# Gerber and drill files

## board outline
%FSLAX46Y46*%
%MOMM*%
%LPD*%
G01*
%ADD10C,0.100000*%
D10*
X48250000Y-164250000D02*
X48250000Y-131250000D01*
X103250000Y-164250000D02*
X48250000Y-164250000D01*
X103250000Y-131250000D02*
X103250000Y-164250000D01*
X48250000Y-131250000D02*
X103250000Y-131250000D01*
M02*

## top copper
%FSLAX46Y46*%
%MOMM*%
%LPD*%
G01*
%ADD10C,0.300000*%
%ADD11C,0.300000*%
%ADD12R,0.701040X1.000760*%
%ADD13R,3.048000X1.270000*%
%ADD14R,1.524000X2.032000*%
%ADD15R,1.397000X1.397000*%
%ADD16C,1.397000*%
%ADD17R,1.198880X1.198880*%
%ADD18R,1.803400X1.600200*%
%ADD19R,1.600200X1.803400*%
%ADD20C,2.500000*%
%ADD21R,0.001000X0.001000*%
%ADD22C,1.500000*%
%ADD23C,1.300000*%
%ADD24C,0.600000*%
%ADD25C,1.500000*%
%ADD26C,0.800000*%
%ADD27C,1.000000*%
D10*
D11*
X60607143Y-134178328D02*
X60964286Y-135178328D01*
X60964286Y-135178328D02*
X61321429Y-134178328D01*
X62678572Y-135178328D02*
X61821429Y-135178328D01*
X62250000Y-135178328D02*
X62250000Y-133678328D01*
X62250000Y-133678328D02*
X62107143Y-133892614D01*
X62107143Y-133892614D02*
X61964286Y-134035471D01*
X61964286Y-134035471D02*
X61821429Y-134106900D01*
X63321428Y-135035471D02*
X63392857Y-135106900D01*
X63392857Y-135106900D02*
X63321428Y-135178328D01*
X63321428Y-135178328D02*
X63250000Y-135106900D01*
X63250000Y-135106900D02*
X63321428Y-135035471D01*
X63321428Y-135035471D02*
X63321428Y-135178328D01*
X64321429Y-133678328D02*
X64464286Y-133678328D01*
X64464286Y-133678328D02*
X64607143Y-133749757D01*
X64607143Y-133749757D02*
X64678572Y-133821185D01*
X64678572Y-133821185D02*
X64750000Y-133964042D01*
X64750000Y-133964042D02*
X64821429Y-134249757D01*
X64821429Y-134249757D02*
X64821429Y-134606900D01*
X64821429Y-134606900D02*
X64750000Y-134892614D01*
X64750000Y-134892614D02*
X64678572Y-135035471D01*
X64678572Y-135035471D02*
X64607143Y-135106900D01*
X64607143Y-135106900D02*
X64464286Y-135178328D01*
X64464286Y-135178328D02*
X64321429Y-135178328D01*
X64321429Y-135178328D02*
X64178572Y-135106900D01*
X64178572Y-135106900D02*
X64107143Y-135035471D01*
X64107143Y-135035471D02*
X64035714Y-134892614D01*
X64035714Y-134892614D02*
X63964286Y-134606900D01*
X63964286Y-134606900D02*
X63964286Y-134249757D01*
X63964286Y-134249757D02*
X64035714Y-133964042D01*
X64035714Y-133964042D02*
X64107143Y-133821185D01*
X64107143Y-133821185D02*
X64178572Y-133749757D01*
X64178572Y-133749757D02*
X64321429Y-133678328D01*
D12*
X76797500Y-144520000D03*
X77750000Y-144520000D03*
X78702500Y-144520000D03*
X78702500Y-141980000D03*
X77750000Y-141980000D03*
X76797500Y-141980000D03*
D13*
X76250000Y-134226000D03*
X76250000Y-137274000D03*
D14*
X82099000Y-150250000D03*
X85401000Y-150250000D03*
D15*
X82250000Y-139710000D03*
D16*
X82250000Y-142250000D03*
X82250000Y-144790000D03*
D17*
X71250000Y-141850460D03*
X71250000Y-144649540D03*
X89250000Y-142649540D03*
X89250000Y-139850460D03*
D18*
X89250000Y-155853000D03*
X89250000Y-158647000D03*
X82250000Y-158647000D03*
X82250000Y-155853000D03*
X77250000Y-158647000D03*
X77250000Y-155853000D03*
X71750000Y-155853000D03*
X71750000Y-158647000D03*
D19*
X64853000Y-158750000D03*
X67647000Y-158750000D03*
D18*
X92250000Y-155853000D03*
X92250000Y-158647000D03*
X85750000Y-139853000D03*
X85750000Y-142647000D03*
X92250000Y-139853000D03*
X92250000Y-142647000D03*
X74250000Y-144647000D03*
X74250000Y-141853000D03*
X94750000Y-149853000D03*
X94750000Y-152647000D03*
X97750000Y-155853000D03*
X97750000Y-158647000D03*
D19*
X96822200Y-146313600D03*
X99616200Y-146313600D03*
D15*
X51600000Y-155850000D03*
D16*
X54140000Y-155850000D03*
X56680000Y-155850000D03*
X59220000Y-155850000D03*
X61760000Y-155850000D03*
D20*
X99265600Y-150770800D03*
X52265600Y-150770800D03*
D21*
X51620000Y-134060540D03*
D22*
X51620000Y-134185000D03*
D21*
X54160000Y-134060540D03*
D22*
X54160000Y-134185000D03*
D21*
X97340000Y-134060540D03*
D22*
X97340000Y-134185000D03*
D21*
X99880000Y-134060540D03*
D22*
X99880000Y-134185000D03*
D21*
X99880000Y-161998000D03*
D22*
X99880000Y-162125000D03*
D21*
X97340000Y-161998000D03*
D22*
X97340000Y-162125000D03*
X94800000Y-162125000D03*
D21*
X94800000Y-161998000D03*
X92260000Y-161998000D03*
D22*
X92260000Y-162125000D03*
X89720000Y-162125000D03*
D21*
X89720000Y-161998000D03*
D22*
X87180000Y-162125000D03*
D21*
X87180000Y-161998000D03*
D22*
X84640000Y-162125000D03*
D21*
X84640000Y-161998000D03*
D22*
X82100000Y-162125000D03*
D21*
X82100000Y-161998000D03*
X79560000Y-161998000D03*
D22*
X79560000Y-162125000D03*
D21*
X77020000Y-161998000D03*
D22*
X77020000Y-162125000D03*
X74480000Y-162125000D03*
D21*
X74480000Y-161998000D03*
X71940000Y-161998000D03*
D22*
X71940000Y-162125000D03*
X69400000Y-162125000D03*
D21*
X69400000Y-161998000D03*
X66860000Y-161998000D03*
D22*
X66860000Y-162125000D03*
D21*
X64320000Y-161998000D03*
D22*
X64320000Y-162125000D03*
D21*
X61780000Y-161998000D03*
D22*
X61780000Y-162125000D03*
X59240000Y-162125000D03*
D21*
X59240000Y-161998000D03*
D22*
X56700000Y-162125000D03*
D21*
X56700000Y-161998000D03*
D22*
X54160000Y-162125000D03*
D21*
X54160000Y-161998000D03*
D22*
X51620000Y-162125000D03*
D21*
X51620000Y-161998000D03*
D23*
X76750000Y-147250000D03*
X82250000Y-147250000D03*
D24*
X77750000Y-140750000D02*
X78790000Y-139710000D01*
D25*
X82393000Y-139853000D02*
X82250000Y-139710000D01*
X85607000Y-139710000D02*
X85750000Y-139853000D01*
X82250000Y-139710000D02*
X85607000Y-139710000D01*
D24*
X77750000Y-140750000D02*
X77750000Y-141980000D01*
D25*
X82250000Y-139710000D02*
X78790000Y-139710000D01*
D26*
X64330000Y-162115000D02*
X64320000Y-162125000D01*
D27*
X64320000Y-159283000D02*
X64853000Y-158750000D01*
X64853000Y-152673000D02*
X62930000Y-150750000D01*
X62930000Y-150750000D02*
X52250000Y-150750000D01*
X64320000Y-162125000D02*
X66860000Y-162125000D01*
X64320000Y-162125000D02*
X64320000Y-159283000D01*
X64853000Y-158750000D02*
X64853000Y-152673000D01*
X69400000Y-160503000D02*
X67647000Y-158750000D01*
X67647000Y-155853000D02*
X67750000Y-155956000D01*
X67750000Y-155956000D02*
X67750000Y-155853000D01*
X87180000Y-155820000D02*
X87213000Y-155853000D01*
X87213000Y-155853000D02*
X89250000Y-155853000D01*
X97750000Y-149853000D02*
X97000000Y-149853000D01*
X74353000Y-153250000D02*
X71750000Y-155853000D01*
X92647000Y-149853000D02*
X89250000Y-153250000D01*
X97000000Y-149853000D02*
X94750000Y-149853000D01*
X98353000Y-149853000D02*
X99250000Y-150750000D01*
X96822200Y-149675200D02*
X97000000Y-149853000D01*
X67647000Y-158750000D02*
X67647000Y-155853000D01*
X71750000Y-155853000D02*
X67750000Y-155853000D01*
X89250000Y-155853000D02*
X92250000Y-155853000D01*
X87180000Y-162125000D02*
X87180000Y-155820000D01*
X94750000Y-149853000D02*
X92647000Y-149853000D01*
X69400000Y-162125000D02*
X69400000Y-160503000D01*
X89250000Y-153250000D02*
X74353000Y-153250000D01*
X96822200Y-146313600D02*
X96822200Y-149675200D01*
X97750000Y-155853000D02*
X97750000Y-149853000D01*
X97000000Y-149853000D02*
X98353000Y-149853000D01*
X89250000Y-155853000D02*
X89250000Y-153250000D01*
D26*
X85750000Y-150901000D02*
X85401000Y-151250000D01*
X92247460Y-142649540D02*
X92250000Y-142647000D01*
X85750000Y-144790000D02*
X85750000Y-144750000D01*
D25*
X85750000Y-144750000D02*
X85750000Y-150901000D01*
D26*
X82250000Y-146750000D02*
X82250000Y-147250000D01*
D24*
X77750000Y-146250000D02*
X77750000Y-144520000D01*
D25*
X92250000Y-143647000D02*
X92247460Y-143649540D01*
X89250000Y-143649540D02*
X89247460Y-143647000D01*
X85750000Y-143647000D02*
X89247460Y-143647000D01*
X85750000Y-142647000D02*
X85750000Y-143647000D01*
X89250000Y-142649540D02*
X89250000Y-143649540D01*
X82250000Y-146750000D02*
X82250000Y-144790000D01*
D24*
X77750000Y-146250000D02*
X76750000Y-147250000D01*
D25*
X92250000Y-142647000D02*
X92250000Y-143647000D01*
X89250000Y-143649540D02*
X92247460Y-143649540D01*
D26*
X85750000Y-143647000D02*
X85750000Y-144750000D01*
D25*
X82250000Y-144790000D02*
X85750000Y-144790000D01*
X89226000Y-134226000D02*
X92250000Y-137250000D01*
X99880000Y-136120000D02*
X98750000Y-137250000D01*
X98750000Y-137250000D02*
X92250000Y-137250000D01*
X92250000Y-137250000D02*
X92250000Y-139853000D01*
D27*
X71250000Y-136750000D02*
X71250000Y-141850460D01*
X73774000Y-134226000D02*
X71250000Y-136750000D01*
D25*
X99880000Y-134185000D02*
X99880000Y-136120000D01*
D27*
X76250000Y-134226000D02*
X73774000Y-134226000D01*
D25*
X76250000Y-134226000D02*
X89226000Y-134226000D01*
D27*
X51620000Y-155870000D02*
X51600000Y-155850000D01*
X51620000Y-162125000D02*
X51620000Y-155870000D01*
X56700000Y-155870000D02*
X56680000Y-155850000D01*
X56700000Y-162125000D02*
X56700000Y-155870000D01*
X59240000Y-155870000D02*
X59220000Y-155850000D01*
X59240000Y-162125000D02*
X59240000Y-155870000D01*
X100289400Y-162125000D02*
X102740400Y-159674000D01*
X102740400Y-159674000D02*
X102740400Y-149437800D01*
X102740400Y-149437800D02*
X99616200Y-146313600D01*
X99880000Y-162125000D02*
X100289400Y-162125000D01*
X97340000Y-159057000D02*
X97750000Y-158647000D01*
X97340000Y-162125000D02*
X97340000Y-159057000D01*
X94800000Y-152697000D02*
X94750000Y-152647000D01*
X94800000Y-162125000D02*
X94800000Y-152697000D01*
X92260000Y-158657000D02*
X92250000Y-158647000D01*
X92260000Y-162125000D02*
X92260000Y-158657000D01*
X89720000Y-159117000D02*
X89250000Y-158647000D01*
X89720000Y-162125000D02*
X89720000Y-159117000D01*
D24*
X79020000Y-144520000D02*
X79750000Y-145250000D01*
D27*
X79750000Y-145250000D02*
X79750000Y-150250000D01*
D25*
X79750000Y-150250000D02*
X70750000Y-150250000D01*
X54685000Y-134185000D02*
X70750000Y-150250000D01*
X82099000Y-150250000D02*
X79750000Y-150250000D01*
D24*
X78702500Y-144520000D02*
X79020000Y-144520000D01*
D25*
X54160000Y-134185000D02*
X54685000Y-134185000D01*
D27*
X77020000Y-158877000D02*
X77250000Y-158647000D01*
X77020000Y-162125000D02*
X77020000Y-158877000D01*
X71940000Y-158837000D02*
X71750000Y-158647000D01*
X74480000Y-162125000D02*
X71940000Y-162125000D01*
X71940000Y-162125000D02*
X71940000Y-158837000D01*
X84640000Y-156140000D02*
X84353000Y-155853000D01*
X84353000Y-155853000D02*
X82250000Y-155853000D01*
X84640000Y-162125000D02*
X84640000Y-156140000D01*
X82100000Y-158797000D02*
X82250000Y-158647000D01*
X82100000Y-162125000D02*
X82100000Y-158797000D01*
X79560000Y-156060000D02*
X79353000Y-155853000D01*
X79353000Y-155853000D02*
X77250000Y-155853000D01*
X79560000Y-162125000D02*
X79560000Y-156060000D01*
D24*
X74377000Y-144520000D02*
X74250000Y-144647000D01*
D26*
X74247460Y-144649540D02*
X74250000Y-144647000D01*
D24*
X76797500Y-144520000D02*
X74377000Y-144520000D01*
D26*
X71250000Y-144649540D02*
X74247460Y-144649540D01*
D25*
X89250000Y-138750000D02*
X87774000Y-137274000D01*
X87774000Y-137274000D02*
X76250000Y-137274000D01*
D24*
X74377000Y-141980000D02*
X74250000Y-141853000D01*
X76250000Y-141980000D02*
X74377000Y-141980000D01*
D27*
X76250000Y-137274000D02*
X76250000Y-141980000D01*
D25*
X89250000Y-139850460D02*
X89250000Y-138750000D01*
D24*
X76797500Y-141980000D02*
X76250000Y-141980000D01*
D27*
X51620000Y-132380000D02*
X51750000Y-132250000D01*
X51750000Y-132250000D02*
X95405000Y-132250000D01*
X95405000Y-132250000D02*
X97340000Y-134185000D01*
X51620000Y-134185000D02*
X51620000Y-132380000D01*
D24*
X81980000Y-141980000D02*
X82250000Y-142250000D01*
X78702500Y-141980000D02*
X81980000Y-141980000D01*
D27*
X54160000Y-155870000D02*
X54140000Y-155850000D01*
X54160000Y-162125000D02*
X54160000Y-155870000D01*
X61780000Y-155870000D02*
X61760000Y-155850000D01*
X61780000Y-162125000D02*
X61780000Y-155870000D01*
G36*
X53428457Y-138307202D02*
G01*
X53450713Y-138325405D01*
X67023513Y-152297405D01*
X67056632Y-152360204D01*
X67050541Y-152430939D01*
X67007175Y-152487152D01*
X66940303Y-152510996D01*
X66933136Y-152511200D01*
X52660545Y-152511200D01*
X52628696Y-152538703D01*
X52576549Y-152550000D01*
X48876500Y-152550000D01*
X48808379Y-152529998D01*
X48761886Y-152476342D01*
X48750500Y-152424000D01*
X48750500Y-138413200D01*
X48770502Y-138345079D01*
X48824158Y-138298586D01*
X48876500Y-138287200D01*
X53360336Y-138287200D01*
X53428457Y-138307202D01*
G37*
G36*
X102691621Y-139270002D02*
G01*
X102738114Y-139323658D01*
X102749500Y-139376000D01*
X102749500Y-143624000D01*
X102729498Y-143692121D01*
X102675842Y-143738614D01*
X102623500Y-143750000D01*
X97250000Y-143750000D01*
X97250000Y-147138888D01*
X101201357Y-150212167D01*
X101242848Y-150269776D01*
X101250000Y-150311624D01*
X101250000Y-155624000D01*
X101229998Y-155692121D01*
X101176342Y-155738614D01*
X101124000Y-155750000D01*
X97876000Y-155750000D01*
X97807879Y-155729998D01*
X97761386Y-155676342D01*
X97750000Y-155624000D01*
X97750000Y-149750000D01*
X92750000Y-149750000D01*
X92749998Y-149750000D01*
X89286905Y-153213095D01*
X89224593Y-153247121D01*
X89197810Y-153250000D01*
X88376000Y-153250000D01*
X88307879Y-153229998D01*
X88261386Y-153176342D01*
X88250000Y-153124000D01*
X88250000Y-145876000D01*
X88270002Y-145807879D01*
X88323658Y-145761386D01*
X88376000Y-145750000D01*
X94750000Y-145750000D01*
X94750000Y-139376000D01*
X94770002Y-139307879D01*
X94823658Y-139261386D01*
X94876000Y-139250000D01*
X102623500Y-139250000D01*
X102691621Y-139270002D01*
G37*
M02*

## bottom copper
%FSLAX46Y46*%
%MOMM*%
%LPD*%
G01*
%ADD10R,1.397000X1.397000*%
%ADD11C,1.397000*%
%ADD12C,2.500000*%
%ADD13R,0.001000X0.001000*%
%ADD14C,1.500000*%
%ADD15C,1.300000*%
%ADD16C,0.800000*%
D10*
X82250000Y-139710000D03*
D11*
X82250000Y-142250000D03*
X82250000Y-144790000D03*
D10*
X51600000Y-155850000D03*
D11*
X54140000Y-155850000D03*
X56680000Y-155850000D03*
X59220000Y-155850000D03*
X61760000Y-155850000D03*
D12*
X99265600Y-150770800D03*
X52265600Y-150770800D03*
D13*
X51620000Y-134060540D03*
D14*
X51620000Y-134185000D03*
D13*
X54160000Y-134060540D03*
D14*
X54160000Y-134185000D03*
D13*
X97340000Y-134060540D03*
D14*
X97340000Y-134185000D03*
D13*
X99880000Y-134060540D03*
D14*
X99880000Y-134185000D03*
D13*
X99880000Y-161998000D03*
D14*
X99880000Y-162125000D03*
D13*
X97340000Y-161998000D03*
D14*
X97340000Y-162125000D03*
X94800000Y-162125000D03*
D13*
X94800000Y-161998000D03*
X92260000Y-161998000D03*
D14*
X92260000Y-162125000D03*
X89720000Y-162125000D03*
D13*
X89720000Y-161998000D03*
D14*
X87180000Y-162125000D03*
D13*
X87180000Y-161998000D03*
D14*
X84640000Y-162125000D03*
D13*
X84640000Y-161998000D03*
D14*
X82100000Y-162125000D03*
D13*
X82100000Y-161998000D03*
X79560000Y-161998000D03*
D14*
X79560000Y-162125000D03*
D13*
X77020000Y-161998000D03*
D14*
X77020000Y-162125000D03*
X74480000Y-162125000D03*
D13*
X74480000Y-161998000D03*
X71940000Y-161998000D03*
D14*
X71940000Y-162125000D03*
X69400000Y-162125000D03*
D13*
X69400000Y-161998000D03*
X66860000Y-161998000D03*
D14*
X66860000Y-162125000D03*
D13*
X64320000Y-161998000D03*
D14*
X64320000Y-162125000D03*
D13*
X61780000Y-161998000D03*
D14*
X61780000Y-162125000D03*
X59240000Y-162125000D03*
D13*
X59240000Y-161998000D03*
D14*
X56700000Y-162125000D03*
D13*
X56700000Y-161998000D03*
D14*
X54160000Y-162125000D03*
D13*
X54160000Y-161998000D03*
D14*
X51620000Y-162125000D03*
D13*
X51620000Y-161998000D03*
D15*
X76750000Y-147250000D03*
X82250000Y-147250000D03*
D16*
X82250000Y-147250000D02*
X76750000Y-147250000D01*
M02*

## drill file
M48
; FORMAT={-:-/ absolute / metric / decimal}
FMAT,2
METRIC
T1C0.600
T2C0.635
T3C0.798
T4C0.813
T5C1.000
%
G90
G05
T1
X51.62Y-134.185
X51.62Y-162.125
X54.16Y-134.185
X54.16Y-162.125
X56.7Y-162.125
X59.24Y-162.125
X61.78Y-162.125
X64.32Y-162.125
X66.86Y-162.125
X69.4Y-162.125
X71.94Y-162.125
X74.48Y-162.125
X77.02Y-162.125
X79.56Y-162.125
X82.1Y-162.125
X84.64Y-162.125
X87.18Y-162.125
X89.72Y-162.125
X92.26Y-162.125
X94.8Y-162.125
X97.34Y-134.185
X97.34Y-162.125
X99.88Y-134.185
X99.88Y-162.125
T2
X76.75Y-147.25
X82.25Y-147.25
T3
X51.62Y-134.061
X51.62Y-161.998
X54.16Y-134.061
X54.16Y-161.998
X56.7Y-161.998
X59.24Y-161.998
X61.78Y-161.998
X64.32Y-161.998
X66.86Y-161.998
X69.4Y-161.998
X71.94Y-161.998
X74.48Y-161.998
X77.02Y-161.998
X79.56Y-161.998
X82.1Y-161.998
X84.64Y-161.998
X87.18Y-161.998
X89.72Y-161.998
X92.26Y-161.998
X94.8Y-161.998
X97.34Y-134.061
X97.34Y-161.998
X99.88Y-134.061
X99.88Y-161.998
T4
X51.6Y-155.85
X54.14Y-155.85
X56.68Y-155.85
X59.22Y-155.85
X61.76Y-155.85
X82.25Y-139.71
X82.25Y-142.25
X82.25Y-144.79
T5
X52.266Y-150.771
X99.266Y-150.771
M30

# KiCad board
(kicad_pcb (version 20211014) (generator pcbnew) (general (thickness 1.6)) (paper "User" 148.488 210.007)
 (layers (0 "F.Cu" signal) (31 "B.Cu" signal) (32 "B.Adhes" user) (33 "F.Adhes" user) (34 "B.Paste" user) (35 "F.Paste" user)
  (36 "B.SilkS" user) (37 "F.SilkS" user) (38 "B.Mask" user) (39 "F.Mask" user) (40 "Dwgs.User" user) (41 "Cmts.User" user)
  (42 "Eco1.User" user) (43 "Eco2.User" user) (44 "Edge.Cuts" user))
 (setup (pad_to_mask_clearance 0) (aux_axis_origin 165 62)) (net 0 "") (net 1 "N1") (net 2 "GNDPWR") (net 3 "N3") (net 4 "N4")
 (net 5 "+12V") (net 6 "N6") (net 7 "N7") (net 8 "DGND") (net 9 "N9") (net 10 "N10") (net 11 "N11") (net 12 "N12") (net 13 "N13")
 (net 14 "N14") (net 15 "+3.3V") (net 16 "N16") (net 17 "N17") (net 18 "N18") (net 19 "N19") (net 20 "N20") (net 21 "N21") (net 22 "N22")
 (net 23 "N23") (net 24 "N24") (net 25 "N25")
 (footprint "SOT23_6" (layer "F.Cu") (at 77.75 143.25)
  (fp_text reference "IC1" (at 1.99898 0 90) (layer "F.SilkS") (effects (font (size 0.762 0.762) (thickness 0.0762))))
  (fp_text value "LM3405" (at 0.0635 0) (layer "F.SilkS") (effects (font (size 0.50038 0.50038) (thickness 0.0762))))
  (pad "1" smd rect locked (at -0.9525 1.27) (size 0.70104 1.00076) (layers "F.Cu" "F.Paste" "F.Mask") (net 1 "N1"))
  (pad "2" smd rect locked (at 0 1.27) (size 0.70104 1.00076) (layers "F.Cu" "F.Paste" "F.Mask") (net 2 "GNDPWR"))
  (pad "3" smd rect locked (at 0.9525 1.27) (size 0.70104 1.00076) (layers "F.Cu" "F.Paste" "F.Mask") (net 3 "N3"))
  (pad "4" smd rect locked (at 0.9525 -1.27) (size 0.70104 1.00076) (layers "F.Cu" "F.Paste" "F.Mask") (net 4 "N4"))
  (pad "5" smd rect locked (at 0 -1.27) (size 0.70104 1.00076) (layers "F.Cu" "F.Paste" "F.Mask") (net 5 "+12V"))
  (pad "6" smd rect locked (at -0.9525 -1.27) (size 0.70104 1.00076) (layers "F.Cu" "F.Paste" "F.Mask") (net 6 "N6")))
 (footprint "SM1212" (layer "F.Cu") (at 76.25 135.75 -90)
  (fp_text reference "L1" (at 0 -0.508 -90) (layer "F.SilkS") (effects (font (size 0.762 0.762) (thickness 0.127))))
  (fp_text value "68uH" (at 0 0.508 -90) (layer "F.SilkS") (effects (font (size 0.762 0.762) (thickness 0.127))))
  (pad "1" smd rect locked (at -1.524 0 270) (size 1.27 3.048) (layers "F.Cu" "F.Paste" "F.Mask") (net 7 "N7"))
  (pad "2" smd rect locked (at 1.524 0 270) (size 1.27 3.048) (layers "F.Cu" "F.Paste" "F.Mask") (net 6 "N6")))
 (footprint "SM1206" (layer "F.Cu") (at 83.75 150.25)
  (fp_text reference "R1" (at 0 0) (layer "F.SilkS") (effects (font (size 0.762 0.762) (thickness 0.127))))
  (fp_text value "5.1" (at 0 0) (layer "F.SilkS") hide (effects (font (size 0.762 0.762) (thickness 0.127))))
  (pad "1" smd rect locked (at -1.651 0) (size 1.524 2.032) (layers "F.Cu" "F.Paste" "F.Mask") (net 3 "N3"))
  (pad "2" smd rect locked (at 1.651 0) (size 1.524 2.032) (layers "F.Cu" "F.Paste" "F.Mask") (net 2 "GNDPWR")))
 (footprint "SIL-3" (layer "F.Cu") (at 82.25 142.25 -90)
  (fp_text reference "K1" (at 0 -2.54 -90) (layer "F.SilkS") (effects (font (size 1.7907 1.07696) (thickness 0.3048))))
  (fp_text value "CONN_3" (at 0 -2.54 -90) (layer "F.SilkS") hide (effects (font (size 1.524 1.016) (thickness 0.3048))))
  (pad "1" thru_hole rect locked (at -2.54 0 270) (size 1.397 1.397) (drill 0.8128) (layers *.Cu *.Mask "F.SilkS") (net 5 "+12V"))
  (pad "2" thru_hole circle locked (at 0 0 270) (size 1.397 1.397) (drill 0.8128) (layers *.Cu *.Mask "F.SilkS") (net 4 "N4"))
  (pad "3" thru_hole circle locked (at 2.54 0 270) (size 1.397 1.397) (drill 0.8128) (layers *.Cu *.Mask "F.SilkS") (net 2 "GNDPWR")))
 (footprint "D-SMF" (layer "F.Cu") (at 71.25 143.25 -90)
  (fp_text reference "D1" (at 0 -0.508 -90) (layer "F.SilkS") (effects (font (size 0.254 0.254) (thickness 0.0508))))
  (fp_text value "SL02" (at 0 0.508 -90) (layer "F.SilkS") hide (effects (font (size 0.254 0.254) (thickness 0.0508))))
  (pad "1" smd rect locked (at -1.39954 0 270) (size 1.19888 1.19888) (layers "F.Cu" "F.Paste" "F.Mask") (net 7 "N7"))
  (pad "2" smd rect locked (at 1.39954 0 270) (size 1.19888 1.19888) (layers "F.Cu" "F.Paste" "F.Mask") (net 1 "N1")))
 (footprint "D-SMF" (layer "F.Cu") (at 89.25 141.25 90)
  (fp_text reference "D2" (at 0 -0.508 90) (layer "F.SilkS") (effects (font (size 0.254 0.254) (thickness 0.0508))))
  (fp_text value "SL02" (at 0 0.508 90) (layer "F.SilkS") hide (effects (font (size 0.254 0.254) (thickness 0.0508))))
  (pad "1" smd rect locked (at -1.39954 0 90) (size 1.19888 1.19888) (layers "F.Cu" "F.Paste" "F.Mask") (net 2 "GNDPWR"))
  (pad "2" smd rect locked (at 1.39954 0 90) (size 1.19888 1.19888) (layers "F.Cu" "F.Paste" "F.Mask") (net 6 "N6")))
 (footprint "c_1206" (layer "F.Cu") (at 89.25 157.25 90)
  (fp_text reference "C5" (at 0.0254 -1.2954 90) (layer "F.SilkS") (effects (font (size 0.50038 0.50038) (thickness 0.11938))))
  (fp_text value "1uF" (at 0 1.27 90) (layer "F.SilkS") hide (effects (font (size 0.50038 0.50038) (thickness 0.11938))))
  (pad "1" smd rect locked (at 1.397 0 90) (size 1.6002 1.8034) (layers "F.Cu" "F.Paste" "F.Mask") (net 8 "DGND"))
  (pad "2" smd rect locked (at -1.397 0 90) (size 1.6002 1.8034) (layers "F.Cu" "F.Paste" "F.Mask") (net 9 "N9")))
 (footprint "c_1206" (layer "F.Cu") (at 82.25 157.25 -90)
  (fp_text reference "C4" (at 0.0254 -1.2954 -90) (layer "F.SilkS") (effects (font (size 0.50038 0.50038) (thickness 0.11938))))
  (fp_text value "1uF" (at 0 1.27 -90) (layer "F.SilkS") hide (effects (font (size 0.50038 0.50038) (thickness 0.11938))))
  (pad "1" smd rect locked (at 1.397 0 270) (size 1.6002 1.8034) (layers "F.Cu" "F.Paste" "F.Mask") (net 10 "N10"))
  (pad "2" smd rect locked (at -1.397 0 270) (size 1.6002 1.8034) (layers "F.Cu" "F.Paste" "F.Mask") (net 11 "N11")))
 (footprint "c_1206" (layer "F.Cu") (at 77.25 157.25 -90)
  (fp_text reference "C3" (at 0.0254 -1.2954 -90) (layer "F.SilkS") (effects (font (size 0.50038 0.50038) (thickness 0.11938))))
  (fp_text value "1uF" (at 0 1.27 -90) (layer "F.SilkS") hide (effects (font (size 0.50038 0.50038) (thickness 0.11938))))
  (pad "1" smd rect locked (at 1.397 0 270) (size 1.6002 1.8034) (layers "F.Cu" "F.Paste" "F.Mask") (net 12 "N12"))
  (pad "2" smd rect locked (at -1.397 0 270) (size 1.6002 1.8034) (layers "F.Cu" "F.Paste" "F.Mask") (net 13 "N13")))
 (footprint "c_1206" (layer "F.Cu") (at 71.75 157.25 90)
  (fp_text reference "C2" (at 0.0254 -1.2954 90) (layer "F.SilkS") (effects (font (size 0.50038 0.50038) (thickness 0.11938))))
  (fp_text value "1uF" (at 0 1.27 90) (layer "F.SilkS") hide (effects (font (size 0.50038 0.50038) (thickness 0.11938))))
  (pad "1" smd rect locked (at 1.397 0 90) (size 1.6002 1.8034) (layers "F.Cu" "F.Paste" "F.Mask") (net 8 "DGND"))
  (pad "2" smd rect locked (at -1.397 0 90) (size 1.6002 1.8034) (layers "F.Cu" "F.Paste" "F.Mask") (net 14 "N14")))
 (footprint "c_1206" (layer "F.Cu") (at 66.25 158.75 180)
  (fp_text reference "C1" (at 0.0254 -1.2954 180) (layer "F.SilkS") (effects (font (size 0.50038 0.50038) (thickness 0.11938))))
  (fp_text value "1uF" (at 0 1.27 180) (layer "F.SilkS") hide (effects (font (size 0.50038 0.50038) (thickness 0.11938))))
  (pad "1" smd rect locked (at 1.397 0 180) (size 1.6002 1.8034) (layers "F.Cu" "F.Paste" "F.Mask") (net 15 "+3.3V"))
  (pad "2" smd rect locked (at -1.397 0 180) (size 1.6002 1.8034) (layers "F.Cu" "F.Paste" "F.Mask") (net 8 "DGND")))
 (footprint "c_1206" (layer "F.Cu") (at 92.25 157.25 90)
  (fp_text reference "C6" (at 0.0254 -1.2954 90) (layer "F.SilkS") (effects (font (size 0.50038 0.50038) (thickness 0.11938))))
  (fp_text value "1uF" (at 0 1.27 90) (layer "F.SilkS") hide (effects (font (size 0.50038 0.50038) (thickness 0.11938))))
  (pad "1" smd rect locked (at 1.397 0 90) (size 1.6002 1.8034) (layers "F.Cu" "F.Paste" "F.Mask") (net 8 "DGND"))
  (pad "2" smd rect locked (at -1.397 0 90) (size 1.6002 1.8034) (layers "F.Cu" "F.Paste" "F.Mask") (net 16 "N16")))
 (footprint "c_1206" (layer "F.Cu") (at 85.75 141.25 90)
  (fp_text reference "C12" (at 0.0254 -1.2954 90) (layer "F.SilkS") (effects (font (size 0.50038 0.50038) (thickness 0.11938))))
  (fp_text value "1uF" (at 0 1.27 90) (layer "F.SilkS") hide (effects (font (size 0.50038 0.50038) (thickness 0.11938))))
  (pad "1" smd rect locked (at 1.397 0 90) (size 1.6002 1.8034) (layers "F.Cu" "F.Paste" "F.Mask") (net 5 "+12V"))
  (pad "2" smd rect locked (at -1.397 0 90) (size 1.6002 1.8034) (layers "F.Cu" "F.Paste" "F.Mask") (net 2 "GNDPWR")))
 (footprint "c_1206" (layer "F.Cu") (at 92.25 141.25 90)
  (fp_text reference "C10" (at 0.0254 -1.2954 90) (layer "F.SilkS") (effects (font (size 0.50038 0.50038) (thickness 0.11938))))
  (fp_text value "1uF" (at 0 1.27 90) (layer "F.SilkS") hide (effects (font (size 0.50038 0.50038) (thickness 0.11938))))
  (pad "1" smd rect locked (at 1.397 0 90) (size 1.6002 1.8034) (layers "F.Cu" "F.Paste" "F.Mask") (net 7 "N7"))
  (pad "2" smd rect locked (at -1.397 0 90) (size 1.6002 1.8034) (layers "F.Cu" "F.Paste" "F.Mask") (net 2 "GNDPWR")))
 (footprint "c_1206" (layer "F.Cu") (at 74.25 143.25 -90)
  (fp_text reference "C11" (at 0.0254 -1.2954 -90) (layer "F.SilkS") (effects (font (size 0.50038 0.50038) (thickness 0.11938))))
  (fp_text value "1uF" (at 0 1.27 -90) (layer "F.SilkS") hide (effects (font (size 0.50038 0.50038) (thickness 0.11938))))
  (pad "1" smd rect locked (at 1.397 0 270) (size 1.6002 1.8034) (layers "F.Cu" "F.Paste" "F.Mask") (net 1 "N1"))
  (pad "2" smd rect locked (at -1.397 0 270) (size 1.6002 1.8034) (layers "F.Cu" "F.Paste" "F.Mask") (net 6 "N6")))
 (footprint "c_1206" (layer "F.Cu") (at 94.75 151.25 90)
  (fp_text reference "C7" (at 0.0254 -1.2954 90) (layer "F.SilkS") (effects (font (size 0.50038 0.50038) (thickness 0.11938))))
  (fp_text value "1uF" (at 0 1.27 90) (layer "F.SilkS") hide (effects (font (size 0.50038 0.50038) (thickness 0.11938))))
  (pad "1" smd rect locked (at 1.397 0 90) (size 1.6002 1.8034) (layers "F.Cu" "F.Paste" "F.Mask") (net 8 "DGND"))
  (pad "2" smd rect locked (at -1.397 0 90) (size 1.6002 1.8034) (layers "F.Cu" "F.Paste" "F.Mask") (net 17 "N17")))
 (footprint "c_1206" (layer "F.Cu") (at 97.75 157.25 90)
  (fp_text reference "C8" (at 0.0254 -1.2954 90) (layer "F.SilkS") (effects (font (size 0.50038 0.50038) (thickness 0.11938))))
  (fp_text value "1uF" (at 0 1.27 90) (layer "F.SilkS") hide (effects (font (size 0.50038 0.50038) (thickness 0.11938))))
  (pad "1" smd rect locked (at 1.397 0 90) (size 1.6002 1.8034) (layers "F.Cu" "F.Paste" "F.Mask") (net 8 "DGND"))
  (pad "2" smd rect locked (at -1.397 0 90) (size 1.6002 1.8034) (layers "F.Cu" "F.Paste" "F.Mask") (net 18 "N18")))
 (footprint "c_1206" (layer "F.Cu") (at 98.2192 146.3136 180)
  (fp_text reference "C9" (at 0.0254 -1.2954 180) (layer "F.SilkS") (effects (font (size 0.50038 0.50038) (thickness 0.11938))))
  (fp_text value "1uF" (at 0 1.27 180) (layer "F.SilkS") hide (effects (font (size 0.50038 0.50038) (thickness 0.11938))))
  (pad "1" smd rect locked (at 1.397 0 180) (size 1.6002 1.8034) (layers "F.Cu" "F.Paste" "F.Mask") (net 8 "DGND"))
  (pad "2" smd rect locked (at -1.397 0 180) (size 1.6002 1.8034) (layers "F.Cu" "F.Paste" "F.Mask") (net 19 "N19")))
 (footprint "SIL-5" (layer "F.Cu") (at 57.95 155.85)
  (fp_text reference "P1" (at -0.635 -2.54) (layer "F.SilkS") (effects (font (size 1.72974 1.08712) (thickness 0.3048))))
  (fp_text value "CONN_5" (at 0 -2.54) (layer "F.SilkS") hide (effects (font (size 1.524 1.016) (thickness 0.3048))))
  (pad "1" thru_hole rect locked (at -6.35 0) (size 1.397 1.397) (drill 0.8128) (layers *.Cu *.Mask "F.SilkS") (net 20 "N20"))
  (pad "2" thru_hole circle locked (at -3.81 0) (size 1.397 1.397) (drill 0.8128) (layers *.Cu *.Mask "F.SilkS") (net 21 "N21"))
  (pad "3" thru_hole circle locked (at -1.27 0) (size 1.397 1.397) (drill 0.8128) (layers *.Cu *.Mask "F.SilkS") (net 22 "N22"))
  (pad "4" thru_hole circle locked (at 1.27 0) (size 1.397 1.397) (drill 0.8128) (layers *.Cu *.Mask "F.SilkS") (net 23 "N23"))
  (pad "5" thru_hole circle locked (at 3.81 0) (size 1.397 1.397) (drill 0.8128) (layers *.Cu *.Mask "F.SilkS") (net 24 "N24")))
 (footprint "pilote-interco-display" (layer "F.Cu") (at 75.7656 146.7708 180)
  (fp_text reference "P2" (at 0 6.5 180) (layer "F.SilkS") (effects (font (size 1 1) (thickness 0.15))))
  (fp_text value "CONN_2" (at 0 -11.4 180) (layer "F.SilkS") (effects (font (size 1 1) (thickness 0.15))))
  (pad "1" thru_hole circle locked (at -23.5 -4 180) (size 2.5 2.5) (drill 1) (layers *.Cu *.Mask "F.SilkS") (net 8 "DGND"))
  (pad "2" thru_hole circle locked (at 23.5 -4 180) (size 2.5 2.5) (drill 1) (layers *.Cu *.Mask "F.SilkS") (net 15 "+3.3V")))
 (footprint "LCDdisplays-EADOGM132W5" (layer "B.Cu") (at 75.75 146.25)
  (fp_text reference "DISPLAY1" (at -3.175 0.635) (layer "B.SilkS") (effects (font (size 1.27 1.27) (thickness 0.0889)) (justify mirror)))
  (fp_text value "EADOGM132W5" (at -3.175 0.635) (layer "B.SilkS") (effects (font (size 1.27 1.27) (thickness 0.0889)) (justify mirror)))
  (pad "1" thru_hole rect locked (at -24.13 -12.18946) (size 1.30556 0) (drill 0.79756) (layers *.Cu "B.Paste" "B.SilkS" "B.Mask")
   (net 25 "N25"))
  (pad "1" thru_hole circle locked (at -24.13 -12.065) (size 1.5 1.5) (drill 0.6) (layers *.Cu *.Mask "B.SilkS") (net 25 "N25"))
  (pad "2" thru_hole rect locked (at -21.59 -12.18946) (size 1.30556 0) (drill 0.79756) (layers *.Cu "B.Paste" "B.SilkS" "B.Mask")
   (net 3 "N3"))
  (pad "2" thru_hole circle locked (at -21.59 -12.065) (size 1.5 1.5) (drill 0.6) (layers *.Cu *.Mask "B.SilkS") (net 3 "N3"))
  (pad "19" thru_hole rect locked (at 21.59 -12.18946) (size 1.30556 0) (drill 0.79756) (layers *.Cu "B.Paste" "B.SilkS" "B.Mask")
   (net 25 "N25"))
  (pad "19" thru_hole circle locked (at 21.59 -12.065) (size 1.5 1.5) (drill 0.6) (layers *.Cu *.Mask "B.SilkS") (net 25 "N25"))
  (pad "20" thru_hole rect locked (at 24.13 -12.18946) (size 1.30556 0) (drill 0.79756) (layers *.Cu "B.Paste" "B.SilkS" "B.Mask")
   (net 7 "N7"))
  (pad "20" thru_hole circle locked (at 24.13 -12.065) (size 1.5 1.5) (drill 0.6) (layers *.Cu *.Mask "B.SilkS") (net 7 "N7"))
  (pad "21" thru_hole rect locked (at 24.13 15.748) (size 1.30556 0) (drill 0.79756) (layers *.Cu "B.Paste" "B.SilkS" "B.Mask")
   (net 19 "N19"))
  (pad "21" thru_hole circle locked (at 24.13 15.875) (size 1.5 1.5) (drill 0.6) (layers *.Cu *.Mask "B.SilkS") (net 19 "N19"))
  (pad "22" thru_hole rect locked (at 21.59 15.748) (size 1.30556 0) (drill 0.79756) (layers *.Cu "B.Paste" "B.SilkS" "B.Mask")
   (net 18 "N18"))
  (pad "22" thru_hole circle locked (at 21.59 15.875) (size 1.5 1.5) (drill 0.6) (layers *.Cu *.Mask "B.SilkS") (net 18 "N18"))
  (pad "23" thru_hole circle locked (at 19.05 15.875) (size 1.5 1.5) (drill 0.6) (layers *.Cu *.Mask "B.SilkS") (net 17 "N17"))
  (pad "23" thru_hole rect locked (at 19.05 15.748) (size 1.30556 0) (drill 0.79756) (layers *.Cu "B.Paste" "B.SilkS" "B.Mask")
   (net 17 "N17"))
  (pad "24" thru_hole rect locked (at 16.51 15.748) (size 1.30556 0) (drill 0.79756) (layers *.Cu "B.Paste" "B.SilkS" "B.Mask")
   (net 16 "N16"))
  (pad "24" thru_hole circle locked (at 16.51 15.875) (size 1.5 1.5) (drill 0.6) (layers *.Cu *.Mask "B.SilkS") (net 16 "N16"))
  (pad "25" thru_hole circle locked (at 13.97 15.875) (size 1.5 1.5) (drill 0.6) (layers *.Cu *.Mask "B.SilkS") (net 9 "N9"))
  (pad "25" thru_hole rect locked (at 13.97 15.748) (size 1.30556 0) (drill 0.79756) (layers *.Cu "B.Paste" "B.SilkS" "B.Mask") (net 9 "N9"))
  (pad "26" thru_hole circle locked (at 11.43 15.875) (size 1.5 1.5) (drill 0.6) (layers *.Cu *.Mask "B.SilkS") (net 8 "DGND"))
  (pad "26" thru_hole rect locked (at 11.43 15.748) (size 1.30556 0) (drill 0.79756) (layers *.Cu "B.Paste" "B.SilkS" "B.Mask")
   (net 8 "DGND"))
  (pad "27" thru_hole circle locked (at 8.89 15.875) (size 1.5 1.5) (drill 0.6) (layers *.Cu *.Mask "B.SilkS") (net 11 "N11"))
  (pad "27" thru_hole rect locked (at 8.89 15.748) (size 1.30556 0) (drill 0.79756) (layers *.Cu "B.Paste" "B.SilkS" "B.Mask")
   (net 11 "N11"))
  (pad "28" thru_hole circle locked (at 6.35 15.875) (size 1.5 1.5) (drill 0.6) (layers *.Cu *.Mask "B.SilkS") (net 10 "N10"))
  (pad "28" thru_hole rect locked (at 6.35 15.748) (size 1.30556 0) (drill 0.79756) (layers *.Cu "B.Paste" "B.SilkS" "B.Mask")
   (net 10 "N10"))
  (pad "29" thru_hole rect locked (at 3.81 15.748) (size 1.30556 0) (drill 0.79756) (layers *.Cu "B.Paste" "B.SilkS" "B.Mask")
   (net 13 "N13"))
  (pad "29" thru_hole circle locked (at 3.81 15.875) (size 1.5 1.5) (drill 0.6) (layers *.Cu *.Mask "B.SilkS") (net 13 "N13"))
  (pad "30" thru_hole rect locked (at 1.27 15.748) (size 1.30556 0) (drill 0.79756) (layers *.Cu "B.Paste" "B.SilkS" "B.Mask")
   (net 12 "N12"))
  (pad "30" thru_hole circle locked (at 1.27 15.875) (size 1.5 1.5) (drill 0.6) (layers *.Cu *.Mask "B.SilkS") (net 12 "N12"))
  (pad "31" thru_hole circle locked (at -1.27 15.875) (size 1.5 1.5) (drill 0.6) (layers *.Cu *.Mask "B.SilkS") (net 14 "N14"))
  (pad "31" thru_hole rect locked (at -1.27 15.748) (size 1.30556 0) (drill 0.79756) (layers *.Cu "B.Paste" "B.SilkS" "B.Mask")
   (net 14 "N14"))
  (pad "32" thru_hole rect locked (at -3.81 15.748) (size 1.30556 0) (drill 0.79756) (layers *.Cu "B.Paste" "B.SilkS" "B.Mask")
   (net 14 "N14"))
  (pad "32" thru_hole circle locked (at -3.81 15.875) (size 1.5 1.5) (drill 0.6) (layers *.Cu *.Mask "B.SilkS") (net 14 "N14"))
  (pad "33" thru_hole circle locked (at -6.35 15.875) (size 1.5 1.5) (drill 0.6) (layers *.Cu *.Mask "B.SilkS") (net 8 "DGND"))
  (pad "33" thru_hole rect locked (at -6.35 15.748) (size 1.30556 0) (drill 0.79756) (layers *.Cu "B.Paste" "B.SilkS" "B.Mask")
   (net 8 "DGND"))
  (pad "34" thru_hole rect locked (at -8.89 15.748) (size 1.30556 0) (drill 0.79756) (layers *.Cu "B.Paste" "B.SilkS" "B.Mask")
   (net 15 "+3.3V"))
  (pad "34" thru_hole circle locked (at -8.89 15.875) (size 1.5 1.5) (drill 0.6) (layers *.Cu *.Mask "B.SilkS") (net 15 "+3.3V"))
  (pad "35" thru_hole rect locked (at -11.43 15.748) (size 1.30556 0) (drill 0.79756) (layers *.Cu "B.Paste" "B.SilkS" "B.Mask")
   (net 15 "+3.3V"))
  (pad "35" thru_hole circle locked (at -11.43 15.875) (size 1.5 1.5) (drill 0.6) (layers *.Cu *.Mask "B.SilkS") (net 15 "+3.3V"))
  (pad "36" thru_hole rect locked (at -13.97 15.748) (size 1.30556 0) (drill 0.79756) (layers *.Cu "B.Paste" "B.SilkS" "B.Mask")
   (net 24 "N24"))
  (pad "36" thru_hole circle locked (at -13.97 15.875) (size 1.5 1.5) (drill 0.6) (layers *.Cu *.Mask "B.SilkS") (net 24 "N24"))
  (pad "37" thru_hole circle locked (at -16.51 15.875) (size 1.5 1.5) (drill 0.6) (layers *.Cu *.Mask "B.SilkS") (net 23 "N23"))
  (pad "37" thru_hole rect locked (at -16.51 15.748) (size 1.30556 0) (drill 0.79756) (layers *.Cu "B.Paste" "B.SilkS" "B.Mask")
   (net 23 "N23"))
  (pad "38" thru_hole circle locked (at -19.05 15.875) (size 1.5 1.5) (drill 0.6) (layers *.Cu *.Mask "B.SilkS") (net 22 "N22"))
  (pad "38" thru_hole rect locked (at -19.05 15.748) (size 1.30556 0) (drill 0.79756) (layers *.Cu "B.Paste" "B.SilkS" "B.Mask")
   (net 22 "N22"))
  (pad "39" thru_hole circle locked (at -21.59 15.875) (size 1.5 1.5) (drill 0.6) (layers *.Cu *.Mask "B.SilkS") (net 21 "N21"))
  (pad "39" thru_hole rect locked (at -21.59 15.748) (size 1.30556 0) (drill 0.79756) (layers *.Cu "B.Paste" "B.SilkS" "B.Mask")
   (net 21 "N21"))
  (pad "40" thru_hole circle locked (at -24.13 15.875) (size 1.5 1.5) (drill 0.6) (layers *.Cu *.Mask "B.SilkS") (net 20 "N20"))
  (pad "40" thru_hole rect locked (at -24.13 15.748) (size 1.30556 0) (drill 0.79756) (layers *.Cu "B.Paste" "B.SilkS" "B.Mask")
   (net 20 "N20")))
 (gr_line (start 48.25 164.25) (end 48.25 131.25) (layer "Edge.Cuts") (width 0.1))
 (gr_line (start 103.25 164.25) (end 48.25 164.25) (layer "Edge.Cuts") (width 0.1))
 (gr_line (start 103.25 131.25) (end 103.25 164.25) (layer "Edge.Cuts") (width 0.1))
 (gr_line (start 48.25 131.25) (end 103.25 131.25) (layer "Edge.Cuts") (width 0.1))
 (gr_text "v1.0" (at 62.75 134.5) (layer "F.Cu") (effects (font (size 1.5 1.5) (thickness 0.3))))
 (segment (start 77.75 140.75) (end 78.79 139.71) (width 0.6) (layer "F.Cu") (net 5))
 (segment (start 82.393 139.853) (end 82.25 139.71) (width 1.5) (layer "F.Cu") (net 5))
 (segment (start 85.607 139.71) (end 85.75 139.853) (width 1.5) (layer "F.Cu") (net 5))
 (segment (start 82.25 139.71) (end 85.607 139.71) (width 1.5) (layer "F.Cu") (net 5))
 (segment (start 77.75 140.75) (end 77.75 141.98) (width 0.6) (layer "F.Cu") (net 5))
 (segment (start 82.25 139.71) (end 78.79 139.71) (width 1.5) (layer "F.Cu") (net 5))
 (segment (start 64.33 162.115) (end 64.32 162.125) (width 0.8) (layer "F.Cu") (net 15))
 (segment (start 64.32 159.283) (end 64.853 158.75) (width 1) (layer "F.Cu") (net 15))
 (segment (start 64.853 152.673) (end 62.93 150.75) (width 1) (layer "F.Cu") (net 15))
 (segment (start 62.93 150.75) (end 52.25 150.75) (width 1) (layer "F.Cu") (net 15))
 (segment (start 64.32 162.125) (end 66.86 162.125) (width 1) (layer "F.Cu") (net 15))
 (segment (start 64.32 162.125) (end 64.32 159.283) (width 1) (layer "F.Cu") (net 15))
 (segment (start 64.853 158.75) (end 64.853 152.673) (width 1) (layer "F.Cu") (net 15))
 (segment (start 69.4 160.503) (end 67.647 158.75) (width 1) (layer "F.Cu") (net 8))
 (segment (start 67.647 155.853) (end 67.75 155.956) (width 1) (layer "F.Cu") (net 8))
 (segment (start 67.75 155.956) (end 67.75 155.853) (width 1) (layer "F.Cu") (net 8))
 (segment (start 87.18 155.82) (end 87.213 155.853) (width 1) (layer "F.Cu") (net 8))
 (segment (start 87.213 155.853) (end 89.25 155.853) (width 1) (layer "F.Cu") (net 8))
 (segment (start 97.75 149.853) (end 97 149.853) (width 1) (layer "F.Cu") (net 8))
 (segment (start 74.353 153.25) (end 71.75 155.853) (width 1) (layer "F.Cu") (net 8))
 (segment (start 92.647 149.853) (end 89.25 153.25) (width 1) (layer "F.Cu") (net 8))
 (segment (start 97 149.853) (end 94.75 149.853) (width 1) (layer "F.Cu") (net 8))
 (segment (start 98.353 149.853) (end 99.25 150.75) (width 1) (layer "F.Cu") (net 8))
 (segment (start 96.8222 149.6752) (end 97 149.853) (width 1) (layer "F.Cu") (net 8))
 (segment (start 67.647 158.75) (end 67.647 155.853) (width 1) (layer "F.Cu") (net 8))
 (segment (start 71.75 155.853) (end 67.75 155.853) (width 1) (layer "F.Cu") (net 8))
 (segment (start 89.25 155.853) (end 92.25 155.853) (width 1) (layer "F.Cu") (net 8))
 (segment (start 87.18 162.125) (end 87.18 155.82) (width 1) (layer "F.Cu") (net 8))
 (segment (start 94.75 149.853) (end 92.647 149.853) (width 1) (layer "F.Cu") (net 8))
 (segment (start 69.4 162.125) (end 69.4 160.503) (width 1) (layer "F.Cu") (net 8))
 (segment (start 89.25 153.25) (end 74.353 153.25) (width 1) (layer "F.Cu") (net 8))
 (segment (start 96.8222 146.3136) (end 96.8222 149.6752) (width 1) (layer "F.Cu") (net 8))
 (segment (start 97.75 155.853) (end 97.75 149.853) (width 1) (layer "F.Cu") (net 8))
 (segment (start 97 149.853) (end 98.353 149.853) (width 1) (layer "F.Cu") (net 8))
 (segment (start 89.25 155.853) (end 89.25 153.25) (width 1) (layer "F.Cu") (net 8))
 (segment (start 85.75 150.901) (end 85.401 151.25) (width 0.8) (layer "F.Cu") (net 2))
 (segment (start 92.24746 142.64954) (end 92.25 142.647) (width 0.8) (layer "F.Cu") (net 2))
 (segment (start 85.75 144.79) (end 85.75 144.75) (width 0.8) (layer "F.Cu") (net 2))
 (segment (start 85.75 144.75) (end 85.75 150.901) (width 1.5) (layer "F.Cu") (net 2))
 (segment (start 82.25 146.75) (end 82.25 147.25) (width 0.8) (layer "F.Cu") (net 2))
 (segment (start 77.75 146.25) (end 77.75 144.52) (width 0.6) (layer "F.Cu") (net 2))
 (segment (start 92.25 143.647) (end 92.24746 143.64954) (width 1.5) (layer "F.Cu") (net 2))
 (segment (start 89.25 143.64954) (end 89.24746 143.647) (width 1.5) (layer "F.Cu") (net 2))
 (segment (start 85.75 143.647) (end 89.24746 143.647) (width 1.5) (layer "F.Cu") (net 2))
 (segment (start 85.75 142.647) (end 85.75 143.647) (width 1.5) (layer "F.Cu") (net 2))
 (segment (start 89.25 142.64954) (end 89.25 143.64954) (width 1.5) (layer "F.Cu") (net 2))
 (segment (start 82.25 146.75) (end 82.25 144.79) (width 1.5) (layer "F.Cu") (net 2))
 (segment (start 77.75 146.25) (end 76.75 147.25) (width 0.6) (layer "F.Cu") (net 2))
 (segment (start 92.25 142.647) (end 92.25 143.647) (width 1.5) (layer "F.Cu") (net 2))
 (segment (start 89.25 143.64954) (end 92.24746 143.64954) (width 1.5) (layer "F.Cu") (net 2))
 (segment (start 85.75 143.647) (end 85.75 144.75) (width 0.8) (layer "F.Cu") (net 2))
 (segment (start 82.25 144.79) (end 85.75 144.79) (width 1.5) (layer "F.Cu") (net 2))
 (via (at 76.75 147.25) (size 1.3) (drill 0.635) (layers "F.Cu" "B.Cu") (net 2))
 (via (at 82.25 147.25) (size 1.3) (drill 0.635) (layers "F.Cu" "B.Cu") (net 2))
 (segment (start 82.25 147.25) (end 76.75 147.25) (width 0.8) (layer "B.Cu") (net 2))
 (segment (start 89.226 134.226) (end 92.25 137.25) (width 1.5) (layer "F.Cu") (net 7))
 (segment (start 99.88 136.12) (end 98.75 137.25) (width 1.5) (layer "F.Cu") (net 7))
 (segment (start 98.75 137.25) (end 92.25 137.25) (width 1.5) (layer "F.Cu") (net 7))
 (segment (start 92.25 137.25) (end 92.25 139.853) (width 1.5) (layer "F.Cu") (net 7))
 (segment (start 71.25 136.75) (end 71.25 141.85046) (width 1) (layer "F.Cu") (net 7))
 (segment (start 73.774 134.226) (end 71.25 136.75) (width 1) (layer "F.Cu") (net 7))
 (segment (start 99.88 134.185) (end 99.88 136.12) (width 1.5) (layer "F.Cu") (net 7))
 (segment (start 76.25 134.226) (end 73.774 134.226) (width 1) (layer "F.Cu") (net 7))
 (segment (start 76.25 134.226) (end 89.226 134.226) (width 1.5) (layer "F.Cu") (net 7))
 (segment (start 51.62 155.87) (end 51.6 155.85) (width 1) (layer "F.Cu") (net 20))
 (segment (start 51.62 162.125) (end 51.62 155.87) (width 1) (layer "F.Cu") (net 20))
 (segment (start 56.7 155.87) (end 56.68 155.85) (width 1) (layer "F.Cu") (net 22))
 (segment (start 56.7 162.125) (end 56.7 155.87) (width 1) (layer "F.Cu") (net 22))
 (segment (start 59.24 155.87) (end 59.22 155.85) (width 1) (layer "F.Cu") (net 23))
 (segment (start 59.24 162.125) (end 59.24 155.87) (width 1) (layer "F.Cu") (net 23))
 (segment (start 100.2894 162.125) (end 102.7404 159.674) (width 1) (layer "F.Cu") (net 19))
 (segment (start 102.7404 159.674) (end 102.7404 149.4378) (width 1) (layer "F.Cu") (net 19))
 (segment (start 102.7404 149.4378) (end 99.6162 146.3136) (width 1) (layer "F.Cu") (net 19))
 (segment (start 99.88 162.125) (end 100.2894 162.125) (width 1) (layer "F.Cu") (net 19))
 (segment (start 97.34 159.057) (end 97.75 158.647) (width 1) (layer "F.Cu") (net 18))
 (segment (start 97.34 162.125) (end 97.34 159.057) (width 1) (layer "F.Cu") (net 18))
 (segment (start 94.8 152.697) (end 94.75 152.647) (width 1) (layer "F.Cu") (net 17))
 (segment (start 94.8 162.125) (end 94.8 152.697) (width 1) (layer "F.Cu") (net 17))
 (segment (start 92.26 158.657) (end 92.25 158.647) (width 1) (layer "F.Cu") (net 16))
 (segment (start 92.26 162.125) (end 92.26 158.657) (width 1) (layer "F.Cu") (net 16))
 (segment (start 89.72 159.117) (end 89.25 158.647) (width 1) (layer "F.Cu") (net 9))
 (segment (start 89.72 162.125) (end 89.72 159.117) (width 1) (layer "F.Cu") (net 9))
 (segment (start 79.02 144.52) (end 79.75 145.25) (width 0.6) (layer "F.Cu") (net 3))
 (segment (start 79.75 145.25) (end 79.75 150.25) (width 1) (layer "F.Cu") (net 3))
 (segment (start 79.75 150.25) (end 70.75 150.25) (width 1.5) (layer "F.Cu") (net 3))
 (segment (start 54.685 134.185) (end 70.75 150.25) (width 1.5) (layer "F.Cu") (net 3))
 (segment (start 82.099 150.25) (end 79.75 150.25) (width 1.5) (layer "F.Cu") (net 3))
 (segment (start 78.7025 144.52) (end 79.02 144.52) (width 0.6) (layer "F.Cu") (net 3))
 (segment (start 54.16 134.185) (end 54.685 134.185) (width 1.5) (layer "F.Cu") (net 3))
 (segment (start 77.02 158.877) (end 77.25 158.647) (width 1) (layer "F.Cu") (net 12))
 (segment (start 77.02 162.125) (end 77.02 158.877) (width 1) (layer "F.Cu") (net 12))
 (segment (start 71.94 158.837) (end 71.75 158.647) (width 1) (layer "F.Cu") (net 14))
 (segment (start 74.48 162.125) (end 71.94 162.125) (width 1) (layer "F.Cu") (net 14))
 (segment (start 71.94 162.125) (end 71.94 158.837) (width 1) (layer "F.Cu") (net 14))
 (segment (start 84.64 156.14) (end 84.353 155.853) (width 1) (layer "F.Cu") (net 11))
 (segment (start 84.353 155.853) (end 82.25 155.853) (width 1) (layer "F.Cu") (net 11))
 (segment (start 84.64 162.125) (end 84.64 156.14) (width 1) (layer "F.Cu") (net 11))
 (segment (start 82.1 158.797) (end 82.25 158.647) (width 1) (layer "F.Cu") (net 10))
 (segment (start 82.1 162.125) (end 82.1 158.797) (width 1) (layer "F.Cu") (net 10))
 (segment (start 79.56 156.06) (end 79.353 155.853) (width 1) (layer "F.Cu") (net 13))
 (segment (start 79.353 155.853) (end 77.25 155.853) (width 1) (layer "F.Cu") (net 13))
 (segment (start 79.56 162.125) (end 79.56 156.06) (width 1) (layer "F.Cu") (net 13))
 (segment (start 74.377 144.52) (end 74.25 144.647) (width 0.6) (layer "F.Cu") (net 1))
 (segment (start 74.24746 144.64954) (end 74.25 144.647) (width 0.8) (layer "F.Cu") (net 1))
 (segment (start 76.7975 144.52) (end 74.377 144.52) (width 0.6) (layer "F.Cu") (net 1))
 (segment (start 71.25 144.64954) (end 74.24746 144.64954) (width 0.8) (layer "F.Cu") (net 1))
 (segment (start 89.25 138.75) (end 87.774 137.274) (width 1.5) (layer "F.Cu") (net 6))
 (segment (start 87.774 137.274) (end 76.25 137.274) (width 1.5) (layer "F.Cu") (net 6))
 (segment (start 74.377 141.98) (end 74.25 141.853) (width 0.6) (layer "F.Cu") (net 6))
 (segment (start 76.25 141.98) (end 74.377 141.98) (width 0.6) (layer "F.Cu") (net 6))
 (segment (start 76.25 137.274) (end 76.25 141.98) (width 1) (layer "F.Cu") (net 6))
 (segment (start 89.25 139.85046) (end 89.25 138.75) (width 1.5) (layer "F.Cu") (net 6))
 (segment (start 76.7975 141.98) (end 76.25 141.98) (width 0.6) (layer "F.Cu") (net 6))
 (segment (start 51.62 132.38) (end 51.75 132.25) (width 1) (layer "F.Cu") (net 25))
 (segment (start 51.75 132.25) (end 95.405 132.25) (width 1) (layer "F.Cu") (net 25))
 (segment (start 95.405 132.25) (end 97.34 134.185) (width 1) (layer "F.Cu") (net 25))
 (segment (start 51.62 134.185) (end 51.62 132.38) (width 1) (layer "F.Cu") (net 25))
 (segment (start 81.98 141.98) (end 82.25 142.25) (width 0.6) (layer "F.Cu") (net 4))
 (segment (start 78.7025 141.98) (end 81.98 141.98) (width 0.6) (layer "F.Cu") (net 4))
 (segment (start 54.16 155.87) (end 54.14 155.85) (width 1) (layer "F.Cu") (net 21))
 (segment (start 54.16 162.125) (end 54.16 155.87) (width 1) (layer "F.Cu") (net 21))
 (segment (start 61.78 155.87) (end 61.76 155.85) (width 1) (layer "F.Cu") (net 24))
 (segment (start 61.78 162.125) (end 61.78 155.87) (width 1) (layer "F.Cu") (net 24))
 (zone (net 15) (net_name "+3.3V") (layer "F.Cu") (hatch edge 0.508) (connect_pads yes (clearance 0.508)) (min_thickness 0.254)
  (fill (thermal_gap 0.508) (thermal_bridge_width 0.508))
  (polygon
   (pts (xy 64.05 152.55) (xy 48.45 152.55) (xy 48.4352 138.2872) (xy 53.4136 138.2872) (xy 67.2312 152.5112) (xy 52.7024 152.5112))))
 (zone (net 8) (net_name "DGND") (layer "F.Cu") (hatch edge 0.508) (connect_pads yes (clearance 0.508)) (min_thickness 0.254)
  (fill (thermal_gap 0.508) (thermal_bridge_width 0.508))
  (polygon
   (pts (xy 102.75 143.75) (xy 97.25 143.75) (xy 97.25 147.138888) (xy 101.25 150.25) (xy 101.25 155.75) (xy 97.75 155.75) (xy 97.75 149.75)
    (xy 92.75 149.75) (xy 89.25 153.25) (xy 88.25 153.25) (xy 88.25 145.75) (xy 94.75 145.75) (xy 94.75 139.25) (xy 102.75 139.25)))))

